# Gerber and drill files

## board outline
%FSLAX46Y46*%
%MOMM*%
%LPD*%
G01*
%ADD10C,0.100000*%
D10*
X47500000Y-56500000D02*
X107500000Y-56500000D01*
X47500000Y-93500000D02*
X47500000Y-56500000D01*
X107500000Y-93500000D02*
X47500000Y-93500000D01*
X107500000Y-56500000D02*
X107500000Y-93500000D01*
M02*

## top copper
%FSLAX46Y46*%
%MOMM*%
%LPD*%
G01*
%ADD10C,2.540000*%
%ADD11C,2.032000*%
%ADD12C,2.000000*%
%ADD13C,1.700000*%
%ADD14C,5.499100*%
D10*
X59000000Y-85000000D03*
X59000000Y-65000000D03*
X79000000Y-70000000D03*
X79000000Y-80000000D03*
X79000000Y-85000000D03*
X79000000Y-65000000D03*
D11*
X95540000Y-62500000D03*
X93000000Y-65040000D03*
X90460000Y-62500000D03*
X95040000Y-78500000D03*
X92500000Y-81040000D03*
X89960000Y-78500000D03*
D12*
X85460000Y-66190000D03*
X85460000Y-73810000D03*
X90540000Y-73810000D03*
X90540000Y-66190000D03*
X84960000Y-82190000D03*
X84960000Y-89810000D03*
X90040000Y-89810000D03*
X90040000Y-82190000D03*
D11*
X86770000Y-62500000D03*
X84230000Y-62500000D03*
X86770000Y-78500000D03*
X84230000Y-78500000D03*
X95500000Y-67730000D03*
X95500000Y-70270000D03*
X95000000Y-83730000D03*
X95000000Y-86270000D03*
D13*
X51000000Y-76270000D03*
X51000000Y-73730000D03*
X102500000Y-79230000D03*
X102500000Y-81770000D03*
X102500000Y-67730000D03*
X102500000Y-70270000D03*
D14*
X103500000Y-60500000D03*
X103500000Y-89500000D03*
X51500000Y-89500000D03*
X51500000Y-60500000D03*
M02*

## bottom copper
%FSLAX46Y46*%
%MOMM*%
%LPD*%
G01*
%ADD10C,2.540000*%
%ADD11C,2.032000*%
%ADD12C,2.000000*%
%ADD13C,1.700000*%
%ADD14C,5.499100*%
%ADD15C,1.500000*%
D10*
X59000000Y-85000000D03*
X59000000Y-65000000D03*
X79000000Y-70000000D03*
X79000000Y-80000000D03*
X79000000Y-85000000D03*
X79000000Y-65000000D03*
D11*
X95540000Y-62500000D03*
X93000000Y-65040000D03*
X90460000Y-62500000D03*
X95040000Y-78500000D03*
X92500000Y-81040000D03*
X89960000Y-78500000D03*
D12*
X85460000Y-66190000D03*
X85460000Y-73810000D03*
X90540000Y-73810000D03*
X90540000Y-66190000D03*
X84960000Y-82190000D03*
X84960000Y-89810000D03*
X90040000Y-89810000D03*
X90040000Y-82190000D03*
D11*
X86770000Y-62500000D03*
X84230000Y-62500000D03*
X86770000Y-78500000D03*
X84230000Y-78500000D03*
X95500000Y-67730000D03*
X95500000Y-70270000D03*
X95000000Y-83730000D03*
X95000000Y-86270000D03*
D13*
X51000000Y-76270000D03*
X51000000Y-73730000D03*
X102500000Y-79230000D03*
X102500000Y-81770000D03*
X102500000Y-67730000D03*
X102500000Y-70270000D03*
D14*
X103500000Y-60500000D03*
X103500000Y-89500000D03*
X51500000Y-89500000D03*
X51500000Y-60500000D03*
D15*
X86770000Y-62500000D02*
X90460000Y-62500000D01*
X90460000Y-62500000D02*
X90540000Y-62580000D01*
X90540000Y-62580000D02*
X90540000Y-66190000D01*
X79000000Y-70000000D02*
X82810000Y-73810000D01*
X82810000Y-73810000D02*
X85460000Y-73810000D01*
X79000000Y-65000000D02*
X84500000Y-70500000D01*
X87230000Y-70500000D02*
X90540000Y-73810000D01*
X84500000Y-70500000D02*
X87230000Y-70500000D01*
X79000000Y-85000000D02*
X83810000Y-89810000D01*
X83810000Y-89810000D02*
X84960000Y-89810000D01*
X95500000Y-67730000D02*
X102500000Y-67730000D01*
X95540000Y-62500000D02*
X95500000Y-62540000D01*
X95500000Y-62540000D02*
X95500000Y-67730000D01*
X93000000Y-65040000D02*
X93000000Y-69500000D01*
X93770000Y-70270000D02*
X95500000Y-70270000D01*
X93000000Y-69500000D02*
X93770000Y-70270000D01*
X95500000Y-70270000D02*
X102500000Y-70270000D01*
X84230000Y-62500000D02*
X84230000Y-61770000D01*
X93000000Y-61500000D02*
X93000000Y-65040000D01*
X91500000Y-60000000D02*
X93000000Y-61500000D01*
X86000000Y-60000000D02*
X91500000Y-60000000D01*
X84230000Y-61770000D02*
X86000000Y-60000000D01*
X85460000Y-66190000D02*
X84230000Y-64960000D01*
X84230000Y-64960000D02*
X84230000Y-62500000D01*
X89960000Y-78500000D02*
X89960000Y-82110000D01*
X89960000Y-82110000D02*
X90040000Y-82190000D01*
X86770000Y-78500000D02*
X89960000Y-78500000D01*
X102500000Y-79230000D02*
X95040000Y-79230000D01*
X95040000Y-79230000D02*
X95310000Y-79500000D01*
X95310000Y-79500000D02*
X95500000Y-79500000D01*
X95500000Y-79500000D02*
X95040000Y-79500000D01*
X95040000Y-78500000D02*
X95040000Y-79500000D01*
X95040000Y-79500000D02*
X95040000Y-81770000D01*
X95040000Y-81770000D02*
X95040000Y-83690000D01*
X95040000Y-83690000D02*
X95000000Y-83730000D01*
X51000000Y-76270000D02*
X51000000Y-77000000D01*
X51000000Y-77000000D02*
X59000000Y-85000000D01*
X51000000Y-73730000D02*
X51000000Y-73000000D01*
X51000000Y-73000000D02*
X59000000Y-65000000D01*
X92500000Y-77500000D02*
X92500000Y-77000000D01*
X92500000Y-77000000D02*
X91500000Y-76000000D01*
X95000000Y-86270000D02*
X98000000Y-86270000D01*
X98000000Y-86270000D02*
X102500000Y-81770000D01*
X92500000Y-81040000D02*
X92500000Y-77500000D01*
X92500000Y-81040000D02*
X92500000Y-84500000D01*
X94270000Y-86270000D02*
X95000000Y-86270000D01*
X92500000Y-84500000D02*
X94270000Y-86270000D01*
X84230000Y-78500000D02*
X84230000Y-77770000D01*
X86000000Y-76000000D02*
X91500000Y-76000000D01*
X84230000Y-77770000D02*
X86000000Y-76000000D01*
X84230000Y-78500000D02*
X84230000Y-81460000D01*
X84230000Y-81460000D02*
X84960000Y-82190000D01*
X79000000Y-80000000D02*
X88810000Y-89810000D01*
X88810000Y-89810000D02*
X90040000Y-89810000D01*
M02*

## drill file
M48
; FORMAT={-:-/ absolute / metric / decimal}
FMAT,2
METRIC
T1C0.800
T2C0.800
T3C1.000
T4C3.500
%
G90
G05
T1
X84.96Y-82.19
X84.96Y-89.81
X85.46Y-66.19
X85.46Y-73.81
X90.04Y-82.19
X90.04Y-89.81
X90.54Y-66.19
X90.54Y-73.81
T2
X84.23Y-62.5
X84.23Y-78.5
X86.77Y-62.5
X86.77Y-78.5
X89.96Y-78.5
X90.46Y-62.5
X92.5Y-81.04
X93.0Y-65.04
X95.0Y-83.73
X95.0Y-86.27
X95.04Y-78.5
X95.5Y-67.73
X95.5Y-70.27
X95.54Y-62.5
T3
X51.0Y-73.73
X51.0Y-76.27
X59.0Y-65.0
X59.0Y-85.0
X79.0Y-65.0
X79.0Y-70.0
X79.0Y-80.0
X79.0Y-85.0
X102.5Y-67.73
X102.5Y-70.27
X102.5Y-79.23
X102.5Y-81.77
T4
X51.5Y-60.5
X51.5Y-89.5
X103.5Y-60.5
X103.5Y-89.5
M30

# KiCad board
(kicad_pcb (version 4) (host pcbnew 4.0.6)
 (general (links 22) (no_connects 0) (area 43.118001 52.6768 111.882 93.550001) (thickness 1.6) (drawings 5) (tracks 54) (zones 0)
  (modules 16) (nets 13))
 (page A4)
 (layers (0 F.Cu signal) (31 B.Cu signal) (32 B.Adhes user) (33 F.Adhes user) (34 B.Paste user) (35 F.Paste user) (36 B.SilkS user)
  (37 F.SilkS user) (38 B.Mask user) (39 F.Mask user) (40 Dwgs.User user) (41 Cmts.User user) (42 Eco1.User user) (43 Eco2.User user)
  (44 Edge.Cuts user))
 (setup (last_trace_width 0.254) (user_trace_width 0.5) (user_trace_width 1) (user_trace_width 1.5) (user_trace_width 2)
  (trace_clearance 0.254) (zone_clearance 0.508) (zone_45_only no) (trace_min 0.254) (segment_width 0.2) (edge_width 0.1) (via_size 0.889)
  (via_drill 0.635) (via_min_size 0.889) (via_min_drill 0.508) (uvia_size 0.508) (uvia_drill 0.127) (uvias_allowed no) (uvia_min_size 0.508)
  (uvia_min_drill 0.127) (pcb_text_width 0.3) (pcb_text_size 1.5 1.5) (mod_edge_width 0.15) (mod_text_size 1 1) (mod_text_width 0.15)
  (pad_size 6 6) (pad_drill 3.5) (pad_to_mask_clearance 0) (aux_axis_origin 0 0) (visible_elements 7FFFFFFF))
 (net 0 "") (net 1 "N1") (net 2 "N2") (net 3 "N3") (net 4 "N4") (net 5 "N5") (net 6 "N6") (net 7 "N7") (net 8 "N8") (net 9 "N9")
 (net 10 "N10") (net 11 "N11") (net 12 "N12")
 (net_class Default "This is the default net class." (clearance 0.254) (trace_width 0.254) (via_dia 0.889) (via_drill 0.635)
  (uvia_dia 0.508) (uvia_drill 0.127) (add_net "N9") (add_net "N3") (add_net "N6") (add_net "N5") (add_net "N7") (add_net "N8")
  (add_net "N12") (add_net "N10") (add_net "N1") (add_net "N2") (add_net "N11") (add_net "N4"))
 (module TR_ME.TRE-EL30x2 (layer F.Cu) (at 69 75 90)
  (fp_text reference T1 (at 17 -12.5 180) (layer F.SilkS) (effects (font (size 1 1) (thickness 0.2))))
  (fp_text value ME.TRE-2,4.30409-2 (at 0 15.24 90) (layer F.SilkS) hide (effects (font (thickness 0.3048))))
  (pad 5 thru_hole circle (at -10 -10 90) (size 2.54 2.54) (drill 1) (layers *.Cu *.Mask F.SilkS) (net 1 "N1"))
  (pad 1 thru_hole circle (at 10 -10 90) (size 2.54 2.54) (drill 1) (layers *.Cu *.Mask F.SilkS) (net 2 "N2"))
  (pad 9 thru_hole circle (at 5 10 90) (size 2.54 2.54) (drill 1) (layers *.Cu *.Mask F.SilkS) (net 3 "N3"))
  (pad 7 thru_hole circle (at -5 10 90) (size 2.54 2.54) (drill 1) (layers *.Cu *.Mask F.SilkS) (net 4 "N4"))
  (pad 6 thru_hole circle (at -10 10 90) (size 2.54 2.54) (drill 1) (layers *.Cu *.Mask F.SilkS) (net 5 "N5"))
  (pad 10 thru_hole circle (at 10 10 90) (size 2.54 2.54) (drill 1) (layers *.Cu *.Mask F.SilkS) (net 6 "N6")))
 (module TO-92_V (layer F.Cu) (at 93 62.5 180)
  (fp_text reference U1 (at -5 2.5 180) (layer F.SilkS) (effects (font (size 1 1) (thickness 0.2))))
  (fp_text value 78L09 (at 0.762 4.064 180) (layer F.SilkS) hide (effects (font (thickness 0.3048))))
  (pad 1 thru_hole circle (at -2.54 0 180) (size 2.032 2.032) (drill 0.8001) (layers *.Cu *.Mask F.SilkS) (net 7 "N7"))
  (pad 2 thru_hole circle (at 0 -2.54 180) (size 2.032 2.032) (drill 0.8001) (layers *.Cu *.Mask F.SilkS) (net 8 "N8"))
  (pad 3 thru_hole circle (at 2.54 0 180) (size 2.032 2.032) (drill 0.8001) (layers *.Cu *.Mask F.SilkS) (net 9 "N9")))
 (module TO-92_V (layer F.Cu) (at 92.5 78.5 180)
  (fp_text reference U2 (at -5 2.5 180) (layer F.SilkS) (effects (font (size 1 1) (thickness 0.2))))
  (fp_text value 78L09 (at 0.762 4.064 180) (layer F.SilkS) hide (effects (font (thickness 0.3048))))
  (pad 1 thru_hole circle (at -2.54 0 180) (size 2.032 2.032) (drill 0.8001) (layers *.Cu *.Mask F.SilkS) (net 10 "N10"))
  (pad 2 thru_hole circle (at 0 -2.54 180) (size 2.032 2.032) (drill 0.8001) (layers *.Cu *.Mask F.SilkS) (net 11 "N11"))
  (pad 3 thru_hole circle (at 2.54 0 180) (size 2.032 2.032) (drill 0.8001) (layers *.Cu *.Mask F.SilkS) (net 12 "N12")))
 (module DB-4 (layer F.Cu) (at 88 70)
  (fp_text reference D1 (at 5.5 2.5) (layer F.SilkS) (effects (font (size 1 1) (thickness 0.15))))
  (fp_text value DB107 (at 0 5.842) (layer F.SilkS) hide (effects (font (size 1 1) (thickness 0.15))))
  (pad 1 thru_hole circle (at -2.54 -3.81) (size 2 2) (drill 0.8) (layers *.Cu *.Mask F.SilkS) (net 8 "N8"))
  (pad 2 thru_hole circle (at -2.54 3.81) (size 2 2) (drill 0.8) (layers *.Cu *.Mask F.SilkS) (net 3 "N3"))
  (pad 3 thru_hole circle (at 2.54 3.81) (size 2 2) (drill 0.8) (layers *.Cu *.Mask F.SilkS) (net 6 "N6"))
  (pad 4 thru_hole circle (at 2.54 -3.81) (size 2 2) (drill 0.8) (layers *.Cu *.Mask F.SilkS) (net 9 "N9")))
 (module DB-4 (layer F.Cu) (at 87.5 86)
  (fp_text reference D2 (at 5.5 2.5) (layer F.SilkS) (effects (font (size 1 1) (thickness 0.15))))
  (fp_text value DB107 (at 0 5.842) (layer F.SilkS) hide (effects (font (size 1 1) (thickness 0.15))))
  (pad 1 thru_hole circle (at -2.54 -3.81) (size 2 2) (drill 0.8) (layers *.Cu *.Mask F.SilkS) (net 11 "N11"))
  (pad 2 thru_hole circle (at -2.54 3.81) (size 2 2) (drill 0.8) (layers *.Cu *.Mask F.SilkS) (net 5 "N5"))
  (pad 3 thru_hole circle (at 2.54 3.81) (size 2 2) (drill 0.8) (layers *.Cu *.Mask F.SilkS) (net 4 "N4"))
  (pad 4 thru_hole circle (at 2.54 -3.81) (size 2 2) (drill 0.8) (layers *.Cu *.Mask F.SilkS) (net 12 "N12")))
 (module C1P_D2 (layer F.Cu) (at 85.5 62.5 180)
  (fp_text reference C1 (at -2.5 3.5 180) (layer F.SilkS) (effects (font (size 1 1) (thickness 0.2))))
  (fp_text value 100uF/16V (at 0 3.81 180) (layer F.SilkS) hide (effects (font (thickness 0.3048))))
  (pad 1 thru_hole circle (at -1.27 0 180) (size 2.032 2.032) (drill 0.8001) (layers *.Cu *.Mask F.SilkS) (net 9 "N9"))
  (pad 2 thru_hole circle (at 1.27 0 180) (size 2.032 2.032) (drill 0.8001) (layers *.Cu *.Mask F.SilkS) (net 8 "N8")))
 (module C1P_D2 (layer F.Cu) (at 85.5 78.5 180)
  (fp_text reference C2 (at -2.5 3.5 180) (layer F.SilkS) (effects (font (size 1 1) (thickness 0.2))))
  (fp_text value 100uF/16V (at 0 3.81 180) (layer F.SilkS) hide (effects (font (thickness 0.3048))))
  (pad 1 thru_hole circle (at -1.27 0 180) (size 2.032 2.032) (drill 0.8001) (layers *.Cu *.Mask F.SilkS) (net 12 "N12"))
  (pad 2 thru_hole circle (at 1.27 0 180) (size 2.032 2.032) (drill 0.8001) (layers *.Cu *.Mask F.SilkS) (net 11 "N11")))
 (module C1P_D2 (layer F.Cu) (at 95.5 69 270)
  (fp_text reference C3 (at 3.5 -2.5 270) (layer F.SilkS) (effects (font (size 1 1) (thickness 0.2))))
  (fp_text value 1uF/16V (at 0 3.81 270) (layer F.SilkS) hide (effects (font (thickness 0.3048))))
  (pad 1 thru_hole circle (at -1.27 0 270) (size 2.032 2.032) (drill 0.8001) (layers *.Cu *.Mask F.SilkS) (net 7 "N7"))
  (pad 2 thru_hole circle (at 1.27 0 270) (size 2.032 2.032) (drill 0.8001) (layers *.Cu *.Mask F.SilkS) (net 8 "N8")))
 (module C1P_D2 (layer F.Cu) (at 95 85 270)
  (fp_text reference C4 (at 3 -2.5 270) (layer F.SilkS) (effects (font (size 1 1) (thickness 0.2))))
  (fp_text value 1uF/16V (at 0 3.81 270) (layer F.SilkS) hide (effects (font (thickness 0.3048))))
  (pad 1 thru_hole circle (at -1.27 0 270) (size 2.032 2.032) (drill 0.8001) (layers *.Cu *.Mask F.SilkS) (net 10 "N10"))
  (pad 2 thru_hole circle (at 1.27 0 270) (size 2.032 2.032) (drill 0.8001) (layers *.Cu *.Mask F.SilkS) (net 11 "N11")))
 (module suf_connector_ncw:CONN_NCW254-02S (layer F.Cu) (at 51 75 90)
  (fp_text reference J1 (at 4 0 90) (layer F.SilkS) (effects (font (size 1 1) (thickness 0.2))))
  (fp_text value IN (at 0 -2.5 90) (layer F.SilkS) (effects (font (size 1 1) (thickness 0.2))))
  (pad 1 thru_hole circle (at -1.27 0 90) (size 1.7 1.7) (drill 1) (layers *.Cu *.Mask F.SilkS) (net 1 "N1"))
  (pad 2 thru_hole circle (at 1.27 0 90) (size 1.7 1.7) (drill 1) (layers *.Cu *.Mask F.SilkS) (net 2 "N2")))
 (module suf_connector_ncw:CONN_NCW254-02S (layer F.Cu) (at 102.5 80.5 270)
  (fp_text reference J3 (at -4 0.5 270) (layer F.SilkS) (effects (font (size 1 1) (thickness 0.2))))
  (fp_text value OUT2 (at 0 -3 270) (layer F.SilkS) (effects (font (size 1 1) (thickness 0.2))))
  (pad 1 thru_hole circle (at -1.27 0 270) (size 1.7 1.7) (drill 1) (layers *.Cu *.Mask F.SilkS) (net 10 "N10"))
  (pad 2 thru_hole circle (at 1.27 0 270) (size 1.7 1.7) (drill 1) (layers *.Cu *.Mask F.SilkS) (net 11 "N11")))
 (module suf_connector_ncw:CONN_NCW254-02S (layer F.Cu) (at 102.5 69 270)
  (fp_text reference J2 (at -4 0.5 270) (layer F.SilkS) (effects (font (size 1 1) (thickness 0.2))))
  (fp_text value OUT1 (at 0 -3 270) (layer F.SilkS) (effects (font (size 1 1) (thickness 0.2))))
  (pad 1 thru_hole circle (at -1.27 0 270) (size 1.7 1.7) (drill 1) (layers *.Cu *.Mask F.SilkS) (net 7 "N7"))
  (pad 2 thru_hole circle (at 1.27 0 270) (size 1.7 1.7) (drill 1) (layers *.Cu *.Mask F.SilkS) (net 8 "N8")))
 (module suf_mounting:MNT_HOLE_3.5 (layer F.Cu) (at 103.5 60.5)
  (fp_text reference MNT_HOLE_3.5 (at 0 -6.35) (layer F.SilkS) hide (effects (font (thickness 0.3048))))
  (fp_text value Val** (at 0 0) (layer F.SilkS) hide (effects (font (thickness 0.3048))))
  (pad "" thru_hole circle (at 0 0) (size 5.4991 5.4991) (drill 3.50012) (layers *.Cu *.Mask F.SilkS)))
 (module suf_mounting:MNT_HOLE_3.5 (layer F.Cu) (at 103.5 89.5)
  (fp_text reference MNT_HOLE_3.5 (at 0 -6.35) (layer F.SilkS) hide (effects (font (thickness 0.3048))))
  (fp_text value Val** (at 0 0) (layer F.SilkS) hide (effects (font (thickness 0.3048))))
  (pad "" thru_hole circle (at 0 0) (size 5.4991 5.4991) (drill 3.50012) (layers *.Cu *.Mask F.SilkS)))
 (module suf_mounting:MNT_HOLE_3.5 (layer F.Cu) (at 51.5 89.5)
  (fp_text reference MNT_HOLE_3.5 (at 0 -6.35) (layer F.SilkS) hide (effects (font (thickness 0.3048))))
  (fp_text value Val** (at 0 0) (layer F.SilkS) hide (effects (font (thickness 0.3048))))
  (pad "" thru_hole circle (at 0 0) (size 5.4991 5.4991) (drill 3.50012) (layers *.Cu *.Mask F.SilkS)))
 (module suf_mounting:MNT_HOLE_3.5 (layer F.Cu) (at 51.5 60.5)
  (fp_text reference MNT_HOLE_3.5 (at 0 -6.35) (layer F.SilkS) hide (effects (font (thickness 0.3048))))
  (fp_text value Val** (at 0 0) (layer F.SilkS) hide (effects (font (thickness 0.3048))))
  (pad "" thru_hole circle (at 0 0) (size 5.4991 5.4991) (drill 3.50012) (layers *.Cu *.Mask F.SilkS)))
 (gr_line (start 47.5 56.5) (end 107.5 56.5) (angle 90) (layer Edge.Cuts) (width 0.1))
 (gr_line (start 47.5 93.5) (end 47.5 56.5) (angle 90) (layer Edge.Cuts) (width 0.1))
 (gr_line (start 107.5 93.5) (end 47.5 93.5) (angle 90) (layer Edge.Cuts) (width 0.1))
 (gr_line (start 107.5 56.5) (end 107.5 93.5) (angle 90) (layer Edge.Cuts) (width 0.1))
 (segment (start 86.77 62.5) (end 90.46 62.5) (width 1.5) (layer B.Cu) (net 9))
 (segment (start 90.46 62.5) (end 90.54 62.58) (width 1.5) (layer B.Cu) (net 9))
 (segment (start 90.54 62.58) (end 90.54 66.19) (width 1.5) (layer B.Cu) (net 9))
 (segment (start 79 70) (end 82.81 73.81) (width 1.5) (layer B.Cu) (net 3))
 (segment (start 82.81 73.81) (end 85.46 73.81) (width 1.5) (layer B.Cu) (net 3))
 (segment (start 79 65) (end 84.5 70.5) (width 1.5) (layer B.Cu) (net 6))
 (segment (start 87.23 70.5) (end 90.54 73.81) (width 1.5) (layer B.Cu) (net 6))
 (segment (start 84.5 70.5) (end 87.23 70.5) (width 1.5) (layer B.Cu) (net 6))
 (segment (start 79 85) (end 83.81 89.81) (width 1.5) (layer B.Cu) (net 5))
 (segment (start 83.81 89.81) (end 84.96 89.81) (width 1.5) (layer B.Cu) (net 5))
 (segment (start 95.5 67.73) (end 102.5 67.73) (width 1.5) (layer B.Cu) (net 7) (status 20))
 (segment (start 95.54 62.5) (end 95.5 62.54) (width 1.5) (layer B.Cu) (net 7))
 (segment (start 95.5 62.54) (end 95.5 67.73) (width 1.5) (layer B.Cu) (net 7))
 (segment (start 93 65.04) (end 93 69.5) (width 1.5) (layer B.Cu) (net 8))
 (segment (start 93.77 70.27) (end 95.5 70.27) (width 1.5) (layer B.Cu) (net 8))
 (segment (start 93 69.5) (end 93.77 70.27) (width 1.5) (layer B.Cu) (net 8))
 (segment (start 95.5 70.27) (end 102.5 70.27) (width 1.5) (layer B.Cu) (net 8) (status 20))
 (segment (start 84.23 62.5) (end 84.23 61.77) (width 1.5) (layer B.Cu) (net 8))
 (segment (start 93 61.5) (end 93 65.04) (width 1.5) (layer B.Cu) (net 8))
 (segment (start 91.5 60) (end 93 61.5) (width 1.5) (layer B.Cu) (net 8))
 (segment (start 86 60) (end 91.5 60) (width 1.5) (layer B.Cu) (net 8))
 (segment (start 84.23 61.77) (end 86 60) (width 1.5) (layer B.Cu) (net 8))
 (segment (start 85.46 66.19) (end 84.23 64.96) (width 1.5) (layer B.Cu) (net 8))
 (segment (start 84.23 64.96) (end 84.23 62.5) (width 1.5) (layer B.Cu) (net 8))
 (segment (start 89.96 78.5) (end 89.96 82.11) (width 1.5) (layer B.Cu) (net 12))
 (segment (start 89.96 82.11) (end 90.04 82.19) (width 1.5) (layer B.Cu) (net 12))
 (segment (start 86.77 78.5) (end 89.96 78.5) (width 1.5) (layer B.Cu) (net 12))
 (segment (start 102.5 79.23) (end 95.04 79.23) (width 1.5) (layer B.Cu) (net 10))
 (segment (start 95.04 79.23) (end 95.31 79.5) (width 1.5) (layer B.Cu) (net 10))
 (segment (start 95.31 79.5) (end 95.5 79.5) (width 1.5) (layer B.Cu) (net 10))
 (segment (start 95.5 79.5) (end 95.04 79.5) (width 1.5) (layer B.Cu) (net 10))
 (segment (start 95.04 78.5) (end 95.04 79.5) (width 1.5) (layer B.Cu) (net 10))
 (segment (start 95.04 79.5) (end 95.04 81.77) (width 1.5) (layer B.Cu) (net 10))
 (segment (start 95.04 81.77) (end 95.04 83.69) (width 1.5) (layer B.Cu) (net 10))
 (segment (start 95.04 83.69) (end 95 83.73) (width 1.5) (layer B.Cu) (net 10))
 (segment (start 51 76.27) (end 51 77) (width 1.5) (layer B.Cu) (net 1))
 (segment (start 51 77) (end 59 85) (width 1.5) (layer B.Cu) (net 1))
 (segment (start 51 73.73) (end 51 73) (width 1.5) (layer B.Cu) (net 2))
 (segment (start 51 73) (end 59 65) (width 1.5) (layer B.Cu) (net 2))
 (segment (start 92.5 77.5) (end 92.5 77) (width 1.5) (layer B.Cu) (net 11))
 (segment (start 92.5 77) (end 91.5 76) (width 1.5) (layer B.Cu) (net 11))
 (segment (start 95 86.27) (end 98 86.27) (width 1.5) (layer B.Cu) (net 11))
 (segment (start 98 86.27) (end 102.5 81.77) (width 1.5) (layer B.Cu) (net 11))
 (segment (start 92.5 81.04) (end 92.5 77.5) (width 1.5) (layer B.Cu) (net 11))
 (segment (start 92.5 81.04) (end 92.5 84.5) (width 1.5) (layer B.Cu) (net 11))
 (segment (start 94.27 86.27) (end 95 86.27) (width 1.5) (layer B.Cu) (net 11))
 (segment (start 92.5 84.5) (end 94.27 86.27) (width 1.5) (layer B.Cu) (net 11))
 (segment (start 84.23 78.5) (end 84.23 77.77) (width 1.5) (layer B.Cu) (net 11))
 (segment (start 86 76) (end 91.5 76) (width 1.5) (layer B.Cu) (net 11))
 (segment (start 84.23 77.77) (end 86 76) (width 1.5) (layer B.Cu) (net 11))
 (segment (start 84.23 78.5) (end 84.23 81.46) (width 1.5) (layer B.Cu) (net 11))
 (segment (start 84.23 81.46) (end 84.96 82.19) (width 1.5) (layer B.Cu) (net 11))
 (segment (start 79 80) (end 88.81 89.81) (width 1.5) (layer B.Cu) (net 4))
 (segment (start 88.81 89.81) (end 90.04 89.81) (width 1.5) (layer B.Cu) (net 4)))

